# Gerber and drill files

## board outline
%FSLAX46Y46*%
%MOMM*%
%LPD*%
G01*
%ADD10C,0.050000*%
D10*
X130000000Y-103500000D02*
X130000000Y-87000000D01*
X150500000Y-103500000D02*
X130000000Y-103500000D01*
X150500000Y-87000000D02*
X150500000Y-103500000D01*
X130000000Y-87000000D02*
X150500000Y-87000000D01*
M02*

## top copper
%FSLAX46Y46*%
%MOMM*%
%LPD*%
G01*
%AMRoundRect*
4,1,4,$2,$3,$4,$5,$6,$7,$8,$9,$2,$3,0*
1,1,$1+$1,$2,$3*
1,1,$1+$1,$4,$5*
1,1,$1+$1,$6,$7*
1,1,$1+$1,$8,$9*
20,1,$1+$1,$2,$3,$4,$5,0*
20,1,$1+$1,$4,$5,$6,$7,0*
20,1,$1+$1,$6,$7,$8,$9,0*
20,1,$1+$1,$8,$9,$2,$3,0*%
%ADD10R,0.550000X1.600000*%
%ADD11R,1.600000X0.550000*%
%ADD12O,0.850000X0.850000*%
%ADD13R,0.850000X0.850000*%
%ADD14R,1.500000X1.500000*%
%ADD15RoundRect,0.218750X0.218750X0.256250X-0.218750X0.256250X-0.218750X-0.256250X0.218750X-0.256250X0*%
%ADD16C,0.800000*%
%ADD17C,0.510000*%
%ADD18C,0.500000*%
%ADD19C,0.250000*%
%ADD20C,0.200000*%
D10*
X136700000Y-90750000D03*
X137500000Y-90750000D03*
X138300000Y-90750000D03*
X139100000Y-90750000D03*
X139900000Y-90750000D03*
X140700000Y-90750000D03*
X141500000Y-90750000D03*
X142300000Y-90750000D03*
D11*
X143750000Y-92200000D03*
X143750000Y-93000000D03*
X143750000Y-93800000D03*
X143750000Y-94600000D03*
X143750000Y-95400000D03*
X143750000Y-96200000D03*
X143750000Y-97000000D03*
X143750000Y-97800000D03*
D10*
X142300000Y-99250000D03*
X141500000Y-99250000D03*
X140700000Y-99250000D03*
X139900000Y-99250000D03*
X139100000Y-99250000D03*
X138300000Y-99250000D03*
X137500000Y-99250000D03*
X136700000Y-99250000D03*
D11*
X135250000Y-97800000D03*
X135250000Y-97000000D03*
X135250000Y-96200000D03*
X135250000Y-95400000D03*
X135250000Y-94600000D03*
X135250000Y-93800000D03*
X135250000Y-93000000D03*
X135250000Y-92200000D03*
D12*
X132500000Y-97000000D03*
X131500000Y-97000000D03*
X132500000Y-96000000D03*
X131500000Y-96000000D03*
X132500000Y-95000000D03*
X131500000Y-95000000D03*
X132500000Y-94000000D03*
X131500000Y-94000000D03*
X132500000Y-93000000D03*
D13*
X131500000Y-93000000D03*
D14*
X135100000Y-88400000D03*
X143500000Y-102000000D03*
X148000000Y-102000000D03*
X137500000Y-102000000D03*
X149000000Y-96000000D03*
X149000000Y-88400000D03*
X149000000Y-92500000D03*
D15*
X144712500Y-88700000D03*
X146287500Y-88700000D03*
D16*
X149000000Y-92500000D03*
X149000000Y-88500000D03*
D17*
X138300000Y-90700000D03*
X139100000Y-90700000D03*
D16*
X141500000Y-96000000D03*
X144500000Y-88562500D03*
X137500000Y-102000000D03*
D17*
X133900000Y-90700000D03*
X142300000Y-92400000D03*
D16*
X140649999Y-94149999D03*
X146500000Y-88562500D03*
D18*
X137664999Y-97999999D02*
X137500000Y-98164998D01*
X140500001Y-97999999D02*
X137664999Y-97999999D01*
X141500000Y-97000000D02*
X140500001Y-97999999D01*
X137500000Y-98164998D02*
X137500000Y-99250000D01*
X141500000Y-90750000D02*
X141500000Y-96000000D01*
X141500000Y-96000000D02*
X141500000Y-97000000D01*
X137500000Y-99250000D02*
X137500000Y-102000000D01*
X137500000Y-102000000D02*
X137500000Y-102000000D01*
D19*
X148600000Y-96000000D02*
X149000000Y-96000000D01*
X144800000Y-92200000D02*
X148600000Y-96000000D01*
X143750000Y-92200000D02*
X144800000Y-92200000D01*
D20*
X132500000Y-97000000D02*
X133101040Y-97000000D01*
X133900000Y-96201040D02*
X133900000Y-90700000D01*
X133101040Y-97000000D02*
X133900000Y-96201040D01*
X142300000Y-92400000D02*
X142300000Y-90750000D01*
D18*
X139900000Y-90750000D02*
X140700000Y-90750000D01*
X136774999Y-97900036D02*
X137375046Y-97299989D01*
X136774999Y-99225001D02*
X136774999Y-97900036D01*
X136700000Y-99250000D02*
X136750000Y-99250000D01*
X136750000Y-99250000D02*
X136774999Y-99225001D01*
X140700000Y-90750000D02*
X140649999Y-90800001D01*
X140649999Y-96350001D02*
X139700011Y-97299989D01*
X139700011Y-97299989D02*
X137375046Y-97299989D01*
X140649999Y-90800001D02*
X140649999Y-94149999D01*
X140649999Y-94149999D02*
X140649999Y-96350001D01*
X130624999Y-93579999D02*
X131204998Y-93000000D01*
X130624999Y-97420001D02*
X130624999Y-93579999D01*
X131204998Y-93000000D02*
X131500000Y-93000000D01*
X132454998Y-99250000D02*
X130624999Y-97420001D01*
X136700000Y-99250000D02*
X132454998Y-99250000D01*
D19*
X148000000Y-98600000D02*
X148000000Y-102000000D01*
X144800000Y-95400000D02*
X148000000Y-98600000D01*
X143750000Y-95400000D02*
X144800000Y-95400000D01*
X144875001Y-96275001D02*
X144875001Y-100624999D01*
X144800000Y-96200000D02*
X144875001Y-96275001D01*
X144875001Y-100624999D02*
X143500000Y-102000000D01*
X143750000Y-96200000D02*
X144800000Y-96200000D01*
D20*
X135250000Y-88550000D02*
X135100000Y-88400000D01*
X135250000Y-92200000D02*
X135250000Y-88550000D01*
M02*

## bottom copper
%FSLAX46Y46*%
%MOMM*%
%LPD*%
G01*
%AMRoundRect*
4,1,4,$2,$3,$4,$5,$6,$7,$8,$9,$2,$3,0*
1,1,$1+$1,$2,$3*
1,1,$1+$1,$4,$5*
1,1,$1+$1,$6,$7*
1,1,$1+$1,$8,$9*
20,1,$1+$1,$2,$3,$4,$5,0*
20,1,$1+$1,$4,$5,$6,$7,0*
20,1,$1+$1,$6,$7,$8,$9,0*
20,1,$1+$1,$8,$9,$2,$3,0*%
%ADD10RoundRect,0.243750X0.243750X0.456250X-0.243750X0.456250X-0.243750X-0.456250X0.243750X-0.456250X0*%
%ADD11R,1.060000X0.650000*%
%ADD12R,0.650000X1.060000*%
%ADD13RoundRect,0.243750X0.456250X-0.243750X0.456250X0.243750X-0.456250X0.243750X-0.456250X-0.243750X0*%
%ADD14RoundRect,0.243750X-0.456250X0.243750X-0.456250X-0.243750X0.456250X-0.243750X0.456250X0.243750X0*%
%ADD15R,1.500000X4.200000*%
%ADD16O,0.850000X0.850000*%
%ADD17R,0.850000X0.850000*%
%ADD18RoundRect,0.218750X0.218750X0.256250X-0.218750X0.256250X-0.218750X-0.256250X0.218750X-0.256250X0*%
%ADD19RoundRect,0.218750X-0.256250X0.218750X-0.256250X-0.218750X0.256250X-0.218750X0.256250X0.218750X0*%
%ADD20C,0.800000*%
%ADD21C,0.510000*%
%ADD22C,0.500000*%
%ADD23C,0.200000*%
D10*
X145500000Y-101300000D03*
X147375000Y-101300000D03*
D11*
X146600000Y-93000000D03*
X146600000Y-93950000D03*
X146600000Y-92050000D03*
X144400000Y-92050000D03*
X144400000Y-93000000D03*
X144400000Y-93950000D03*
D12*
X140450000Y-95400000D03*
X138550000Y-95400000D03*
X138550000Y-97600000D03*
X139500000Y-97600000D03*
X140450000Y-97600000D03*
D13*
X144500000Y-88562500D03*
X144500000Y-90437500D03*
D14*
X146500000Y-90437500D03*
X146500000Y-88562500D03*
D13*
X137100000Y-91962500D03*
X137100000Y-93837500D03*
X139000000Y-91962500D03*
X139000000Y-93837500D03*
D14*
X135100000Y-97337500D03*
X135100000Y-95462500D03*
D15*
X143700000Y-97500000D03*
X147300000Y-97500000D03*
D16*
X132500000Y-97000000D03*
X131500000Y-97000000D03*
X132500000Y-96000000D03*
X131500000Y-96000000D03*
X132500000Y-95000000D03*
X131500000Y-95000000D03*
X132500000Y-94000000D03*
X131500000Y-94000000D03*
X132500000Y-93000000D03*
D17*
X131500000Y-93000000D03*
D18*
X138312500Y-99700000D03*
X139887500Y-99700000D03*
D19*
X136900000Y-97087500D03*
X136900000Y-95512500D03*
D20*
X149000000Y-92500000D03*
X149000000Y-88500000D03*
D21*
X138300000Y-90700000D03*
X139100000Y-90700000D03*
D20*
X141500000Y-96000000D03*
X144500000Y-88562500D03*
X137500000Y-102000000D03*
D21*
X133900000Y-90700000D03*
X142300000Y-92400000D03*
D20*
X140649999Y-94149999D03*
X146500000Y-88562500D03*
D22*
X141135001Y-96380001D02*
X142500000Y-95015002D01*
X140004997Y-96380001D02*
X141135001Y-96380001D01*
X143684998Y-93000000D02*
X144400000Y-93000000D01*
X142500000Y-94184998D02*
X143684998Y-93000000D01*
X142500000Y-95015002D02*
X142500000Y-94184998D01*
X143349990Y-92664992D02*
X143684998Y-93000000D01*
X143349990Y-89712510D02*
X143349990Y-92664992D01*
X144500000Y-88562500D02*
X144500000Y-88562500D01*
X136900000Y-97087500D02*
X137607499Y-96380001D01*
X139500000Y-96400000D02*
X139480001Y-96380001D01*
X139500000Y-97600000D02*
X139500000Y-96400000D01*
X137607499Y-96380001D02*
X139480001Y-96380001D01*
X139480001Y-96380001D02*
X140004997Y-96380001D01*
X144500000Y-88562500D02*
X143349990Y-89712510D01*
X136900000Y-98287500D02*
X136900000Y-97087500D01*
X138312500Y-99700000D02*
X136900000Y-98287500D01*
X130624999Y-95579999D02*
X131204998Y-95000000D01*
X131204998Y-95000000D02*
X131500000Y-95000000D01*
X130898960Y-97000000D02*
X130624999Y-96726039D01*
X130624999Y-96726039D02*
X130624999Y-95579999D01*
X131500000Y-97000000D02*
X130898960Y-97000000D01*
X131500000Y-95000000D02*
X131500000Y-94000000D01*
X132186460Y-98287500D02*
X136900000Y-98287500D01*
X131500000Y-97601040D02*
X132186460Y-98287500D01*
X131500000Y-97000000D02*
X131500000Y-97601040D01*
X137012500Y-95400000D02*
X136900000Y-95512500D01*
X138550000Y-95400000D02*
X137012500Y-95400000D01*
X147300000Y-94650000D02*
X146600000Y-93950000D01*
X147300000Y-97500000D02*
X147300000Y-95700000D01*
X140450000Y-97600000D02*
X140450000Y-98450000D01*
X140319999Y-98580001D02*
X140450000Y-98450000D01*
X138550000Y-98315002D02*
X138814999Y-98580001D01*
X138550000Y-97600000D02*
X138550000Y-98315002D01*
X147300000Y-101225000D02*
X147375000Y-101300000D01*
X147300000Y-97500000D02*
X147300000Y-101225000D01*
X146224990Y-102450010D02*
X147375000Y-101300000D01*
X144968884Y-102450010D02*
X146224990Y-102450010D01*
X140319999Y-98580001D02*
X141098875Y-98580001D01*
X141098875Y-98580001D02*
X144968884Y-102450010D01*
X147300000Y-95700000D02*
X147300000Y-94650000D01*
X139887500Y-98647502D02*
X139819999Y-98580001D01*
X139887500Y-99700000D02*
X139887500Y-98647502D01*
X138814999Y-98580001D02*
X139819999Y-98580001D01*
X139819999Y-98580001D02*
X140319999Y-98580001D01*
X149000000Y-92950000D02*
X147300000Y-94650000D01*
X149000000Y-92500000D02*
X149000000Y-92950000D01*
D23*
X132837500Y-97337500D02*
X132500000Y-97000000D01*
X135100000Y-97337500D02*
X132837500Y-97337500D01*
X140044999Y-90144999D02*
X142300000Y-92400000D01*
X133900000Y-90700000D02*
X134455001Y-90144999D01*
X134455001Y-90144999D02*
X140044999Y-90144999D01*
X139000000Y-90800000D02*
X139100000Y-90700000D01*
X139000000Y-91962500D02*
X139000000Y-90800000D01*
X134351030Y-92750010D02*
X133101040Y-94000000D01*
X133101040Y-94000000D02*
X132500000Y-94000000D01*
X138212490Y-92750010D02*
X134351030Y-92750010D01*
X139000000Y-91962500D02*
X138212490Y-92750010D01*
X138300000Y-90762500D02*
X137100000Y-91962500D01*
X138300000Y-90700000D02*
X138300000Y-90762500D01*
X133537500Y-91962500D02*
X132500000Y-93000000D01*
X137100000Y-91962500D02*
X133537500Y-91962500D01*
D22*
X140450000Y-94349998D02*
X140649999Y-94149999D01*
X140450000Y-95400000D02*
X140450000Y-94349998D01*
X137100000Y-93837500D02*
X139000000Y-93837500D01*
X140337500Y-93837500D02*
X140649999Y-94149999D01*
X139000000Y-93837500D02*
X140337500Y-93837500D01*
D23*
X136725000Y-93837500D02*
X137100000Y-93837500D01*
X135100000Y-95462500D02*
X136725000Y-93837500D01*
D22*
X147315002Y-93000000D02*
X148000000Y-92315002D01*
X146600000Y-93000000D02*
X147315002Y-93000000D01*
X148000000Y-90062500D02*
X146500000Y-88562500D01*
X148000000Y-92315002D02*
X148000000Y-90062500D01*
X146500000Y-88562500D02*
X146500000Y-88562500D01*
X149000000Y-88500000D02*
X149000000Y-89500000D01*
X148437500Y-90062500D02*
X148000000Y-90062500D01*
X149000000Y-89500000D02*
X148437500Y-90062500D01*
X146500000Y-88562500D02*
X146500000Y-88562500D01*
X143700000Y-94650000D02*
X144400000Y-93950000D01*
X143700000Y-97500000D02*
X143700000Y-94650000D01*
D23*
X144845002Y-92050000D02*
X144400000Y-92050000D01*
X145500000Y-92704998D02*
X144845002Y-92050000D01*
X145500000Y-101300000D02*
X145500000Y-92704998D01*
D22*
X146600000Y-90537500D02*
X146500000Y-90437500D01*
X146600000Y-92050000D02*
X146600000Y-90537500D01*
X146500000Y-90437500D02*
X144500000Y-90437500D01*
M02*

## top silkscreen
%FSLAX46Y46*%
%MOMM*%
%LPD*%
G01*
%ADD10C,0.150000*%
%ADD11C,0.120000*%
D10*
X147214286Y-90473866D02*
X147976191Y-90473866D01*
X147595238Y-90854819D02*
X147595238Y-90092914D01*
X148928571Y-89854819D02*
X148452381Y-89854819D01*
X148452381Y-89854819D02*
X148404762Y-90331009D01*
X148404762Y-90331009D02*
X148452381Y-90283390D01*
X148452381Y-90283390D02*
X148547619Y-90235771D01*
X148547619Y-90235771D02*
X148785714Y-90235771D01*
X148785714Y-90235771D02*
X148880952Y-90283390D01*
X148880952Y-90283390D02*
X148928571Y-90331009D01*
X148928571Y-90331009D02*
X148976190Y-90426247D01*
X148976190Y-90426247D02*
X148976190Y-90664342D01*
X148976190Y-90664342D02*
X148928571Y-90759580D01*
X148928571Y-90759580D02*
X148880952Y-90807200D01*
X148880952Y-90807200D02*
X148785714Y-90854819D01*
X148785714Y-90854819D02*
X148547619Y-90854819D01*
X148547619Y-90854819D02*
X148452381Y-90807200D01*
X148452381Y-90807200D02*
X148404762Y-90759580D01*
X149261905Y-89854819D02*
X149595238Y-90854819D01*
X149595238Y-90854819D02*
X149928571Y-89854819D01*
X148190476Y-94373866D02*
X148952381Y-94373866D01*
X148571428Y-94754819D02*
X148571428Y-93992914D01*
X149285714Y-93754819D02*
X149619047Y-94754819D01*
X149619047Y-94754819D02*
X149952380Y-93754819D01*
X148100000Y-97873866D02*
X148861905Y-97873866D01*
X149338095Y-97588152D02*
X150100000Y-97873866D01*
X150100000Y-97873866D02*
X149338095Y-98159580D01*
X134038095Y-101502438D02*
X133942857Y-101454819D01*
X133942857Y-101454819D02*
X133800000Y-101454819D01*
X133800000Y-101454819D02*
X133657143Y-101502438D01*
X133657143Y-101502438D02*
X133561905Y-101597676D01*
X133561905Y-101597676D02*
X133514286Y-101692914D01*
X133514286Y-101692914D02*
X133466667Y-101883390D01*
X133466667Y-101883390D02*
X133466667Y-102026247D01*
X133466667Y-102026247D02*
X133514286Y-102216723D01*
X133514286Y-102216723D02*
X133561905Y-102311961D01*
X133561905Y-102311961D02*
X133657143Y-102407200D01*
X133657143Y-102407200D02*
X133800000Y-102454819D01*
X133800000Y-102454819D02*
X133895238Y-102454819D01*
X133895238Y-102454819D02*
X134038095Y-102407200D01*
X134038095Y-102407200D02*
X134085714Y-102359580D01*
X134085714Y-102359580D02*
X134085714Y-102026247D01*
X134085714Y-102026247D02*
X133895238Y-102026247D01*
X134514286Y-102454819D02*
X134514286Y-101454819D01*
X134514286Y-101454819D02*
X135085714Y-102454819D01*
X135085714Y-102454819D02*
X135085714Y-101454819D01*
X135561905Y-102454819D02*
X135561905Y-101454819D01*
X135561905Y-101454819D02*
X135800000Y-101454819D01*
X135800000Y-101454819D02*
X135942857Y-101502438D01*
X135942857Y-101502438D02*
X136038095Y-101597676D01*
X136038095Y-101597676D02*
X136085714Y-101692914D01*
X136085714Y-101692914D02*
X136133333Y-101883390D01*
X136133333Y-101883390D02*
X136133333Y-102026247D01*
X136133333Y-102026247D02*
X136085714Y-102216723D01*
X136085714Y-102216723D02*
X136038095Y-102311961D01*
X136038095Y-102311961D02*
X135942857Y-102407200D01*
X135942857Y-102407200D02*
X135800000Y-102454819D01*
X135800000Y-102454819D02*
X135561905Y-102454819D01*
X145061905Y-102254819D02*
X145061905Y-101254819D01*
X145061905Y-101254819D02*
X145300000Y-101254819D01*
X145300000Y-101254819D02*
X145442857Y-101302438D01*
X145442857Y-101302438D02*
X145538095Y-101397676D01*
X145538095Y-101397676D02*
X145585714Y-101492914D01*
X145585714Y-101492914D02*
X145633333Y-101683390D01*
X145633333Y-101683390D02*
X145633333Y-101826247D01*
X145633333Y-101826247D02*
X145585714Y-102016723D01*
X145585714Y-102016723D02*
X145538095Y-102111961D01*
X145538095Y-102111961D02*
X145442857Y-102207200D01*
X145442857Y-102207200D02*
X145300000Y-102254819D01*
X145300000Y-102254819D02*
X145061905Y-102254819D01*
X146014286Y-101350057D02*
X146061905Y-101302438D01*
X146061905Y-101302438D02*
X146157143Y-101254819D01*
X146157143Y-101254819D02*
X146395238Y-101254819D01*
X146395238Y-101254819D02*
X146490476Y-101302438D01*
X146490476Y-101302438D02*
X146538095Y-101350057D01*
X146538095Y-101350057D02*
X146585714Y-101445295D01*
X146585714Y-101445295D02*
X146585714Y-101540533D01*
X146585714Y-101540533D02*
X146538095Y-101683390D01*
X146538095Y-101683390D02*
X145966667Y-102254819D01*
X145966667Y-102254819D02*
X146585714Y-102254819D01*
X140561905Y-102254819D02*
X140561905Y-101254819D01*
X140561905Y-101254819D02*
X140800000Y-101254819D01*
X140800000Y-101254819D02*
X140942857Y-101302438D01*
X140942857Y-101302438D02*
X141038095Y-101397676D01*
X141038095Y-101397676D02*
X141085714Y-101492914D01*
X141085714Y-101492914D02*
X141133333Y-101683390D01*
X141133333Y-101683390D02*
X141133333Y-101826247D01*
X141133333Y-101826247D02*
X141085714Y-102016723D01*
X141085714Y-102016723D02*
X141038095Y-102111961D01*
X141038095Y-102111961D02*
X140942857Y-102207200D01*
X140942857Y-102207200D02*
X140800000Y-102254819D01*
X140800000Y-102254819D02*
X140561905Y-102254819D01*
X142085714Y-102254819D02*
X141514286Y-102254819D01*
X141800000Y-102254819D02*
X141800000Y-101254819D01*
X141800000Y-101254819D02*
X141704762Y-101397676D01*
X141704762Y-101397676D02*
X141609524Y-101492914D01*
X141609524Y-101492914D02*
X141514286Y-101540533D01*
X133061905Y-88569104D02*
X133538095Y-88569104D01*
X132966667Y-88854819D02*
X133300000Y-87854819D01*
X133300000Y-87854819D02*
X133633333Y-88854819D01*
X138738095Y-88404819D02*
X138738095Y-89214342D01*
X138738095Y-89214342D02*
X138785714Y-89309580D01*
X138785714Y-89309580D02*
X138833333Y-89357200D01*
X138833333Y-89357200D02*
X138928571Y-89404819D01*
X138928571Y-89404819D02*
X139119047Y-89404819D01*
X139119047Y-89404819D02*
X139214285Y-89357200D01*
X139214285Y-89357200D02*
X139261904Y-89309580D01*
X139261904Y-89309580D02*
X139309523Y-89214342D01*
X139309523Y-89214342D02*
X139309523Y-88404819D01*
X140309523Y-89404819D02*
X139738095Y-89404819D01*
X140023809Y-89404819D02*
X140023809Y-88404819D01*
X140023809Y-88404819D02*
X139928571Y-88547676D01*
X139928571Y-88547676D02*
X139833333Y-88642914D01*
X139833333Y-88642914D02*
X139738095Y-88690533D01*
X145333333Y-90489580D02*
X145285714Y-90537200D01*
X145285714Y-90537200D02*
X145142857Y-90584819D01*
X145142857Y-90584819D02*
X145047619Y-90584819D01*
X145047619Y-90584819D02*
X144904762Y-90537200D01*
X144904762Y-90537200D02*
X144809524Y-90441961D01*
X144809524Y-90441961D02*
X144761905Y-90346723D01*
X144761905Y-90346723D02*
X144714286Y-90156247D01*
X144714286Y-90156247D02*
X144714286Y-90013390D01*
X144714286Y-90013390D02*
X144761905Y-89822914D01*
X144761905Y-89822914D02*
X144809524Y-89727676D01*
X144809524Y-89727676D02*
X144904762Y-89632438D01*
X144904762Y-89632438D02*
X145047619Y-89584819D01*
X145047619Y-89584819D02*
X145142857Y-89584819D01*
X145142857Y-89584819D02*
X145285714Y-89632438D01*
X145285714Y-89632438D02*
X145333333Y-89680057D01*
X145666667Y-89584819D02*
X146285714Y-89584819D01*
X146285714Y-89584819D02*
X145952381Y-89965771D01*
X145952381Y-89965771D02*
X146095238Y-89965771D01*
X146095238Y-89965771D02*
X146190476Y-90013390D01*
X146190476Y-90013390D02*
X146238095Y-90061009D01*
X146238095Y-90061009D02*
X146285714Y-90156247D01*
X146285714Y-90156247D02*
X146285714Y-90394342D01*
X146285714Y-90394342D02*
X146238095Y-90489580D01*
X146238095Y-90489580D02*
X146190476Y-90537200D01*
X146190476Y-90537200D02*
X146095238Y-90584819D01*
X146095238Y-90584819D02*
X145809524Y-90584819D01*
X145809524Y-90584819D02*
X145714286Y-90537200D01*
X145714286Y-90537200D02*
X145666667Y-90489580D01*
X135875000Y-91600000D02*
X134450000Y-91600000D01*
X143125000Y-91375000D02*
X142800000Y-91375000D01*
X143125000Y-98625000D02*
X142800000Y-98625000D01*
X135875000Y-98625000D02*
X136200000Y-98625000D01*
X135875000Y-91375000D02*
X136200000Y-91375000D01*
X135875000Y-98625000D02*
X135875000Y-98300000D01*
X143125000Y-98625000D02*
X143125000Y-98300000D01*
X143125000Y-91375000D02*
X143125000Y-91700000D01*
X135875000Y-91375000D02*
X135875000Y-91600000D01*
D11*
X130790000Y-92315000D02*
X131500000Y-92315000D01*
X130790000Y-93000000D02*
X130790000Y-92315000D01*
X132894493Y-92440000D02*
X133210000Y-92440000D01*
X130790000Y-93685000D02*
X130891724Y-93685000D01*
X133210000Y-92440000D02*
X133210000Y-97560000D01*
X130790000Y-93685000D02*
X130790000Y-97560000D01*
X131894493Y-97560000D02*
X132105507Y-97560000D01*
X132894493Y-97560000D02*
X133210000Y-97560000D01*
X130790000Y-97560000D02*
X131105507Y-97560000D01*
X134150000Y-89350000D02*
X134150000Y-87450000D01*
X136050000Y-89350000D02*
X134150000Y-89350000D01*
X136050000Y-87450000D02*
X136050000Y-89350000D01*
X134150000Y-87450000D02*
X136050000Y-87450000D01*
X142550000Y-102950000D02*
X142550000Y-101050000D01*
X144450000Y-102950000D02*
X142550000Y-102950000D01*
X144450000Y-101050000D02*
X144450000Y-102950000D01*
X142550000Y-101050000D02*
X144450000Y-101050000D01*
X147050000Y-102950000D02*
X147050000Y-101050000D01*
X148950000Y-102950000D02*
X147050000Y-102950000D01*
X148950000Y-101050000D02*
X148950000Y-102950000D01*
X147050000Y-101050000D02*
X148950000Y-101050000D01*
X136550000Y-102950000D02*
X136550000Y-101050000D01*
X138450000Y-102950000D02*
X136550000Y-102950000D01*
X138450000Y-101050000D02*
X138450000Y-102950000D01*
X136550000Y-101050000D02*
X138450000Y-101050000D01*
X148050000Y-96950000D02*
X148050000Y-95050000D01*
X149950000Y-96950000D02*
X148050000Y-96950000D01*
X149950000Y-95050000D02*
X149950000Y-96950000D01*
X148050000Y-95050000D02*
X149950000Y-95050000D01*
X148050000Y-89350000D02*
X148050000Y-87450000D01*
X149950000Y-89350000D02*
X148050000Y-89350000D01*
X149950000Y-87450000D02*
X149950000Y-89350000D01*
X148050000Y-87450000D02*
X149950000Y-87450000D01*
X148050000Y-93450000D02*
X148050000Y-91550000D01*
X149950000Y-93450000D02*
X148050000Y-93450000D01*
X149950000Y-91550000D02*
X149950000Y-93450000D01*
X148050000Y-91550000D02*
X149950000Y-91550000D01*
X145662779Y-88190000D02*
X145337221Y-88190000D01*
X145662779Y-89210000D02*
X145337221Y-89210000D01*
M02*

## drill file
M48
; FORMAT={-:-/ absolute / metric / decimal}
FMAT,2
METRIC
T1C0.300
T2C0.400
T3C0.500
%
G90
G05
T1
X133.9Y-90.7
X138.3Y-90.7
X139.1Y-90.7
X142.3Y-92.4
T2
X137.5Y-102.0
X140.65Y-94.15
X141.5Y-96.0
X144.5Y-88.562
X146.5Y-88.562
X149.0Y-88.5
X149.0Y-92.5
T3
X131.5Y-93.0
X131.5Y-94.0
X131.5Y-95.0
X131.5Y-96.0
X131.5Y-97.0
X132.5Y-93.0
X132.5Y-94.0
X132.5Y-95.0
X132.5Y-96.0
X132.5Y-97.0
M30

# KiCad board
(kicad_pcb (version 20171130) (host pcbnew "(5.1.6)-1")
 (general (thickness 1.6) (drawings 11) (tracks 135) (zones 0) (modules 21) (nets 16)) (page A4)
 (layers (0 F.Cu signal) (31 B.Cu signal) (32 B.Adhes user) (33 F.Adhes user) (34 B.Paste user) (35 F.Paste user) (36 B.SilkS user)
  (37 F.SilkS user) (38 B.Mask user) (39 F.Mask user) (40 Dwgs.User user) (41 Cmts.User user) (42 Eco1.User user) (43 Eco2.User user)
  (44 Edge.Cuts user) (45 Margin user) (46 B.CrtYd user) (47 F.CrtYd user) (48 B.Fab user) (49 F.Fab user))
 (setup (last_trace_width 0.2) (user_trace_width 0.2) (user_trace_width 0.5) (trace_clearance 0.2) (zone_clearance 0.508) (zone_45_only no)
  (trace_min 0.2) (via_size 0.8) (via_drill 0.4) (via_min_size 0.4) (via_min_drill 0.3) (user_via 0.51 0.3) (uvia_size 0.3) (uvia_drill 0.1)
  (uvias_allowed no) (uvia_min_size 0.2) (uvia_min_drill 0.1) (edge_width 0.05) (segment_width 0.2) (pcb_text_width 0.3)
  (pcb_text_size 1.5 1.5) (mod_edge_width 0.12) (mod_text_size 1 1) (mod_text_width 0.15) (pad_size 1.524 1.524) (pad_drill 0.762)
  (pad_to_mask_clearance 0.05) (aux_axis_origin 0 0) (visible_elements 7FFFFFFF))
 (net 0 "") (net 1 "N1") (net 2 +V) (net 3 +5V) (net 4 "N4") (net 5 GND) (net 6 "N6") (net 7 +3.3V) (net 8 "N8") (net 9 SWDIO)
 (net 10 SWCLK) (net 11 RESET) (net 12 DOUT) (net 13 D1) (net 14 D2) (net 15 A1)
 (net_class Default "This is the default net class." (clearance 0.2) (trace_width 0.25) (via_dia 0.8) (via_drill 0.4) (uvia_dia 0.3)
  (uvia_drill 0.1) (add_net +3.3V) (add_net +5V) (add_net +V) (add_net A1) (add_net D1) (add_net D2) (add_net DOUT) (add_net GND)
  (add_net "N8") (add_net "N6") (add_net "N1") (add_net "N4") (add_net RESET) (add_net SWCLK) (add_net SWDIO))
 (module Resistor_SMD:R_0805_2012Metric (layer B.Cu) (at 146.4375 101.3 180)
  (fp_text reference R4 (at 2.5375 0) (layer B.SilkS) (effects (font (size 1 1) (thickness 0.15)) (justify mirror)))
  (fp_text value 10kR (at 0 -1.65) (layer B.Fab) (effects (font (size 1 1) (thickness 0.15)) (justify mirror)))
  (pad 2 smd roundrect (at 0.9375 0 180) (size 0.975 1.4) (layers B.Cu B.Paste B.Mask) (roundrect_rratio 0.25) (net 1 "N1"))
  (pad 1 smd roundrect (at -0.9375 0 180) (size 0.975 1.4) (layers B.Cu B.Paste B.Mask) (roundrect_rratio 0.25) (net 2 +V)))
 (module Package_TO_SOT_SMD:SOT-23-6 (layer B.Cu) (at 145.5 93)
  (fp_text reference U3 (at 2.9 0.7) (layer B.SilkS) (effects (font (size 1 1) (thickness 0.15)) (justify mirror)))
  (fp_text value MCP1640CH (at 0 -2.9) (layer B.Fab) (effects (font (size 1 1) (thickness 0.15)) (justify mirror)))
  (pad 5 smd rect (at 1.1 0) (size 1.06 0.65) (layers B.Cu B.Paste B.Mask) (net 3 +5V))
  (pad 6 smd rect (at 1.1 0.95) (size 1.06 0.65) (layers B.Cu B.Paste B.Mask) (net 2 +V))
  (pad 4 smd rect (at 1.1 -0.95) (size 1.06 0.65) (layers B.Cu B.Paste B.Mask) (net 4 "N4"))
  (pad 3 smd rect (at -1.1 -0.95) (size 1.06 0.65) (layers B.Cu B.Paste B.Mask) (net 1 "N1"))
  (pad 2 smd rect (at -1.1 0) (size 1.06 0.65) (layers B.Cu B.Paste B.Mask) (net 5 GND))
  (pad 1 smd rect (at -1.1 0.95) (size 1.06 0.65) (layers B.Cu B.Paste B.Mask) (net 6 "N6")))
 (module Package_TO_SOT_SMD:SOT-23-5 (layer B.Cu) (at 139.5 96.5 90)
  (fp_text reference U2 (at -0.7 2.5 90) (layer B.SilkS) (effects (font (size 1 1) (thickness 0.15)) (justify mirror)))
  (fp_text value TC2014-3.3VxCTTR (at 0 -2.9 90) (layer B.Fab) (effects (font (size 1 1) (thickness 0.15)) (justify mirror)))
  (pad 5 smd rect (at 1.1 0.95 90) (size 1.06 0.65) (layers B.Cu B.Paste B.Mask) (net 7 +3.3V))
  (pad 4 smd rect (at 1.1 -0.95 90) (size 1.06 0.65) (layers B.Cu B.Paste B.Mask) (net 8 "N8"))
  (pad 3 smd rect (at -1.1 -0.95 90) (size 1.06 0.65) (layers B.Cu B.Paste B.Mask) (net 2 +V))
  (pad 2 smd rect (at -1.1 0 90) (size 1.06 0.65) (layers B.Cu B.Paste B.Mask) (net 5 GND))
  (pad 1 smd rect (at -1.1 0.95 90) (size 1.06 0.65) (layers B.Cu B.Paste B.Mask) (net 2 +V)))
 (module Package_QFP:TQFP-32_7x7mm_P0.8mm (layer F.Cu) (at 139.5 95)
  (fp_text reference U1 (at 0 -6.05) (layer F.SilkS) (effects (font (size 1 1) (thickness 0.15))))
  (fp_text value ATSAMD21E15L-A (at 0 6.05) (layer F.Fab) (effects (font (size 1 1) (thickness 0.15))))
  (fp_line (start -3.625 -3.4) (end -5.05 -3.4) (layer F.SilkS) (width 0.15))
  (fp_line (start 3.625 -3.625) (end 3.3 -3.625) (layer F.SilkS) (width 0.15))
  (fp_line (start 3.625 3.625) (end 3.3 3.625) (layer F.SilkS) (width 0.15))
  (fp_line (start -3.625 3.625) (end -3.3 3.625) (layer F.SilkS) (width 0.15))
  (fp_line (start -3.625 -3.625) (end -3.3 -3.625) (layer F.SilkS) (width 0.15))
  (fp_line (start -3.625 3.625) (end -3.625 3.3) (layer F.SilkS) (width 0.15))
  (fp_line (start 3.625 3.625) (end 3.625 3.3) (layer F.SilkS) (width 0.15))
  (fp_line (start 3.625 -3.625) (end 3.625 -3.3) (layer F.SilkS) (width 0.15))
  (fp_line (start -3.625 -3.625) (end -3.625 -3.4) (layer F.SilkS) (width 0.15))
  (pad 32 smd rect (at -2.8 -4.25 90) (size 1.6 0.55) (layers F.Cu F.Paste F.Mask))
  (pad 31 smd rect (at -2 -4.25 90) (size 1.6 0.55) (layers F.Cu F.Paste F.Mask))
  (pad 30 smd rect (at -1.2 -4.25 90) (size 1.6 0.55) (layers F.Cu F.Paste F.Mask) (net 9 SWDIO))
  (pad 29 smd rect (at -0.4 -4.25 90) (size 1.6 0.55) (layers F.Cu F.Paste F.Mask) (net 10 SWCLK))
  (pad 28 smd rect (at 0.4 -4.25 90) (size 1.6 0.55) (layers F.Cu F.Paste F.Mask) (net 7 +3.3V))
  (pad 27 smd rect (at 1.2 -4.25 90) (size 1.6 0.55) (layers F.Cu F.Paste F.Mask) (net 7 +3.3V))
  (pad 26 smd rect (at 2 -4.25 90) (size 1.6 0.55) (layers F.Cu F.Paste F.Mask) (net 5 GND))
  (pad 25 smd rect (at 2.8 -4.25 90) (size 1.6 0.55) (layers F.Cu F.Paste F.Mask) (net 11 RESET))
  (pad 24 smd rect (at 4.25 -2.8) (size 1.6 0.55) (layers F.Cu F.Paste F.Mask) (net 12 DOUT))
  (pad 23 smd rect (at 4.25 -2) (size 1.6 0.55) (layers F.Cu F.Paste F.Mask))
  (pad 22 smd rect (at 4.25 -1.2) (size 1.6 0.55) (layers F.Cu F.Paste F.Mask))
  (pad 21 smd rect (at 4.25 -0.4) (size 1.6 0.55) (layers F.Cu F.Paste F.Mask))
  (pad 20 smd rect (at 4.25 0.4) (size 1.6 0.55) (layers F.Cu F.Paste F.Mask) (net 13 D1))
  (pad 19 smd rect (at 4.25 1.2) (size 1.6 0.55) (layers F.Cu F.Paste F.Mask) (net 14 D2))
  (pad 18 smd rect (at 4.25 2) (size 1.6 0.55) (layers F.Cu F.Paste F.Mask))
  (pad 17 smd rect (at 4.25 2.8) (size 1.6 0.55) (layers F.Cu F.Paste F.Mask))
  (pad 16 smd rect (at 2.8 4.25 90) (size 1.6 0.55) (layers F.Cu F.Paste F.Mask))
  (pad 15 smd rect (at 2 4.25 90) (size 1.6 0.55) (layers F.Cu F.Paste F.Mask))
  (pad 14 smd rect (at 1.2 4.25 90) (size 1.6 0.55) (layers F.Cu F.Paste F.Mask))
  (pad 13 smd rect (at 0.4 4.25 90) (size 1.6 0.55) (layers F.Cu F.Paste F.Mask))
  (pad 12 smd rect (at -0.4 4.25 90) (size 1.6 0.55) (layers F.Cu F.Paste F.Mask))
  (pad 11 smd rect (at -1.2 4.25 90) (size 1.6 0.55) (layers F.Cu F.Paste F.Mask))
  (pad 10 smd rect (at -2 4.25 90) (size 1.6 0.55) (layers F.Cu F.Paste F.Mask) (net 5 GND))
  (pad 9 smd rect (at -2.8 4.25 90) (size 1.6 0.55) (layers F.Cu F.Paste F.Mask) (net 7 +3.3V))
  (pad 8 smd rect (at -4.25 2.8) (size 1.6 0.55) (layers F.Cu F.Paste F.Mask))
  (pad 7 smd rect (at -4.25 2) (size 1.6 0.55) (layers F.Cu F.Paste F.Mask))
  (pad 6 smd rect (at -4.25 1.2) (size 1.6 0.55) (layers F.Cu F.Paste F.Mask))
  (pad 5 smd rect (at -4.25 0.4) (size 1.6 0.55) (layers F.Cu F.Paste F.Mask))
  (pad 4 smd rect (at -4.25 -0.4) (size 1.6 0.55) (layers F.Cu F.Paste F.Mask))
  (pad 3 smd rect (at -4.25 -1.2) (size 1.6 0.55) (layers F.Cu F.Paste F.Mask))
  (pad 2 smd rect (at -4.25 -2) (size 1.6 0.55) (layers F.Cu F.Paste F.Mask))
  (pad 1 smd rect (at -4.25 -2.8) (size 1.6 0.55) (layers F.Cu F.Paste F.Mask) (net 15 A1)))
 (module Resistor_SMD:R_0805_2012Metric (layer B.Cu) (at 144.5 89.5 90)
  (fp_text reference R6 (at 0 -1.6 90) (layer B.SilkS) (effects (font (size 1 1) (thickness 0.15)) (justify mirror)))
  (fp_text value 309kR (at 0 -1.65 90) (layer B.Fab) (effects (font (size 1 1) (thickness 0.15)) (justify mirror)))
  (pad 2 smd roundrect (at 0.9375 0 90) (size 0.975 1.4) (layers B.Cu B.Paste B.Mask) (roundrect_rratio 0.25) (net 5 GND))
  (pad 1 smd roundrect (at -0.9375 0 90) (size 0.975 1.4) (layers B.Cu B.Paste B.Mask) (roundrect_rratio 0.25) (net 4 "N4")))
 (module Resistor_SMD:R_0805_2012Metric (layer B.Cu) (at 146.5 89.5 270)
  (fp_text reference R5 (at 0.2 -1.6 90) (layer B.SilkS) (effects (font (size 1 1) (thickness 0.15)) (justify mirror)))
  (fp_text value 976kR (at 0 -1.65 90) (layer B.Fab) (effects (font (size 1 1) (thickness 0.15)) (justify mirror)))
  (pad 2 smd roundrect (at 0.9375 0 270) (size 0.975 1.4) (layers B.Cu B.Paste B.Mask) (roundrect_rratio 0.25) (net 4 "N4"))
  (pad 1 smd roundrect (at -0.9375 0 270) (size 0.975 1.4) (layers B.Cu B.Paste B.Mask) (roundrect_rratio 0.25) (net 3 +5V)))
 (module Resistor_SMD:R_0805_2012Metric (layer B.Cu) (at 137.1 92.9 90)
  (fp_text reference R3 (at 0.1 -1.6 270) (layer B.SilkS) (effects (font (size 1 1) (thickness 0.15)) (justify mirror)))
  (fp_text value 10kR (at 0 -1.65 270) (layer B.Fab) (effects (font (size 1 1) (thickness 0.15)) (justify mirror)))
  (pad 2 smd roundrect (at 0.9375 0 90) (size 0.975 1.4) (layers B.Cu B.Paste B.Mask) (roundrect_rratio 0.25) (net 9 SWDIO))
  (pad 1 smd roundrect (at -0.9375 0 90) (size 0.975 1.4) (layers B.Cu B.Paste B.Mask) (roundrect_rratio 0.25) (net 7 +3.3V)))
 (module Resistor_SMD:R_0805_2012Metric (layer B.Cu) (at 139 92.9 90)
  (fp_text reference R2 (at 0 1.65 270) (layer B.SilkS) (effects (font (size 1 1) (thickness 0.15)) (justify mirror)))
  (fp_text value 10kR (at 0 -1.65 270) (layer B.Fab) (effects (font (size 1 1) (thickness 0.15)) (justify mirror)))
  (pad 2 smd roundrect (at 0.9375 0 90) (size 0.975 1.4) (layers B.Cu B.Paste B.Mask) (roundrect_rratio 0.25) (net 10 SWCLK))
  (pad 1 smd roundrect (at -0.9375 0 90) (size 0.975 1.4) (layers B.Cu B.Paste B.Mask) (roundrect_rratio 0.25) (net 7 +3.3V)))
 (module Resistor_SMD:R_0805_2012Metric (layer B.Cu) (at 135.1 96.4 270)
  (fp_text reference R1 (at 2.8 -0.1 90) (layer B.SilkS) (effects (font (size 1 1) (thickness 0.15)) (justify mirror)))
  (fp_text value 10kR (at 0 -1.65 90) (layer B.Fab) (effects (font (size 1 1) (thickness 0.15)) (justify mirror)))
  (pad 2 smd roundrect (at 0.9375 0 270) (size 0.975 1.4) (layers B.Cu B.Paste B.Mask) (roundrect_rratio 0.25) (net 11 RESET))
  (pad 1 smd roundrect (at -0.9375 0 270) (size 0.975 1.4) (layers B.Cu B.Paste B.Mask) (roundrect_rratio 0.25) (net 7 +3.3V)))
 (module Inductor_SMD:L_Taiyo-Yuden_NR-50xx (layer B.Cu) (at 145.5 97.5 180)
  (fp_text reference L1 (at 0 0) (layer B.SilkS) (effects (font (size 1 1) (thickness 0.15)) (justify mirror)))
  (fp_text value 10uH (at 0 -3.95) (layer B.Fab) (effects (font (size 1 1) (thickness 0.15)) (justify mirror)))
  (pad 2 smd rect (at 1.8 0 180) (size 1.5 4.2) (layers B.Cu B.Paste B.Mask) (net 6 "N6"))
  (pad 1 smd rect (at -1.8 0 180) (size 1.5 4.2) (layers B.Cu B.Paste B.Mask) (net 2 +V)))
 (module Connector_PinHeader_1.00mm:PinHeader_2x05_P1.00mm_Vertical (layer F.Cu) (at 131.5 93)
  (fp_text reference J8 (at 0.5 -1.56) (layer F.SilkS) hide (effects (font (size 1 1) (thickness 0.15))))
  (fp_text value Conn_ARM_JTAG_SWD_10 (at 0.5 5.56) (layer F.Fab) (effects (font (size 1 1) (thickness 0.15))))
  (fp_line (start -0.71 -0.685) (end 0 -0.685) (layer F.SilkS) (width 0.12))
  (fp_line (start -0.71 0) (end -0.71 -0.685) (layer F.SilkS) (width 0.12))
  (fp_line (start 1.394493 -0.56) (end 1.71 -0.56) (layer F.SilkS) (width 0.12))
  (fp_line (start -0.71 0.685) (end -0.608276 0.685) (layer F.SilkS) (width 0.12))
  (fp_line (start 1.71 -0.56) (end 1.71 4.56) (layer F.SilkS) (width 0.12))
  (fp_line (start -0.71 0.685) (end -0.71 4.56) (layer F.SilkS) (width 0.12))
  (fp_line (start 0.394493 4.56) (end 0.605507 4.56) (layer F.SilkS) (width 0.12))
  (fp_line (start 1.394493 4.56) (end 1.71 4.56) (layer F.SilkS) (width 0.12))
  (fp_line (start -0.71 4.56) (end -0.394493 4.56) (layer F.SilkS) (width 0.12))
  (pad 10 thru_hole oval (at 1 4) (size 0.85 0.85) (drill 0.5) (layers *.Cu *.Mask) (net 11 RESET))
  (pad 9 thru_hole oval (at 0 4) (size 0.85 0.85) (drill 0.5) (layers *.Cu *.Mask) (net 5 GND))
  (pad 8 thru_hole oval (at 1 3) (size 0.85 0.85) (drill 0.5) (layers *.Cu *.Mask))
  (pad 7 thru_hole oval (at 0 3) (size 0.85 0.85) (drill 0.5) (layers *.Cu *.Mask))
  (pad 6 thru_hole oval (at 1 2) (size 0.85 0.85) (drill 0.5) (layers *.Cu *.Mask))
  (pad 5 thru_hole oval (at 0 2) (size 0.85 0.85) (drill 0.5) (layers *.Cu *.Mask) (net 5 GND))
  (pad 4 thru_hole oval (at 1 1) (size 0.85 0.85) (drill 0.5) (layers *.Cu *.Mask) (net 10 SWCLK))
  (pad 3 thru_hole oval (at 0 1) (size 0.85 0.85) (drill 0.5) (layers *.Cu *.Mask) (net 5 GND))
  (pad 2 thru_hole oval (at 1 0) (size 0.85 0.85) (drill 0.5) (layers *.Cu *.Mask) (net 9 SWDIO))
  (pad 1 thru_hole rect (at 0 0) (size 0.85 0.85) (drill 0.5) (layers *.Cu *.Mask) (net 7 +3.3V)))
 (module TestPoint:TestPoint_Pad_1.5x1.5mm (layer F.Cu) (at 135.1 88.4)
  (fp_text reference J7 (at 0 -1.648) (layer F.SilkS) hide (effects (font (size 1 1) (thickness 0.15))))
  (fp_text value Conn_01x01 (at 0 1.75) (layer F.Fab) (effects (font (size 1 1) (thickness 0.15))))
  (fp_line (start -0.95 0.95) (end -0.95 -0.95) (layer F.SilkS) (width 0.12))
  (fp_line (start 0.95 0.95) (end -0.95 0.95) (layer F.SilkS) (width 0.12))
  (fp_line (start 0.95 -0.95) (end 0.95 0.95) (layer F.SilkS) (width 0.12))
  (fp_line (start -0.95 -0.95) (end 0.95 -0.95) (layer F.SilkS) (width 0.12))
  (pad 1 smd rect (at 0 0) (size 1.5 1.5) (layers F.Cu F.Mask) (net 15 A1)))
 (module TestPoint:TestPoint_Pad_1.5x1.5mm (layer F.Cu) (at 143.5 102)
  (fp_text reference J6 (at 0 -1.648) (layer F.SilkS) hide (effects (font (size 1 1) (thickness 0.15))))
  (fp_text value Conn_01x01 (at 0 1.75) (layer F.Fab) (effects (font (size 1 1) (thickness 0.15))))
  (fp_line (start -0.95 0.95) (end -0.95 -0.95) (layer F.SilkS) (width 0.12))
  (fp_line (start 0.95 0.95) (end -0.95 0.95) (layer F.SilkS) (width 0.12))
  (fp_line (start 0.95 -0.95) (end 0.95 0.95) (layer F.SilkS) (width 0.12))
  (fp_line (start -0.95 -0.95) (end 0.95 -0.95) (layer F.SilkS) (width 0.12))
  (pad 1 smd rect (at 0 0) (size 1.5 1.5) (layers F.Cu F.Mask) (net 14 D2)))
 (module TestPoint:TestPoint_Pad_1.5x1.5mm (layer F.Cu) (at 148 102)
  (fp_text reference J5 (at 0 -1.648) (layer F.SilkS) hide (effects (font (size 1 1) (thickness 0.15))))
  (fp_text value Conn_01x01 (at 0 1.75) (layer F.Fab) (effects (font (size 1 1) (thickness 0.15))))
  (fp_line (start -0.95 0.95) (end -0.95 -0.95) (layer F.SilkS) (width 0.12))
  (fp_line (start 0.95 0.95) (end -0.95 0.95) (layer F.SilkS) (width 0.12))
  (fp_line (start 0.95 -0.95) (end 0.95 0.95) (layer F.SilkS) (width 0.12))
  (fp_line (start -0.95 -0.95) (end 0.95 -0.95) (layer F.SilkS) (width 0.12))
  (pad 1 smd rect (at 0 0) (size 1.5 1.5) (layers F.Cu F.Mask) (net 13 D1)))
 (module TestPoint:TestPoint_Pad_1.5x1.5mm (layer F.Cu) (at 137.5 102)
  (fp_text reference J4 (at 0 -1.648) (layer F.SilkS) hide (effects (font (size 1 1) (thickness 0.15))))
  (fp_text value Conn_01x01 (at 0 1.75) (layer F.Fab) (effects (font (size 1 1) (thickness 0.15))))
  (fp_line (start -0.95 0.95) (end -0.95 -0.95) (layer F.SilkS) (width 0.12))
  (fp_line (start 0.95 0.95) (end -0.95 0.95) (layer F.SilkS) (width 0.12))
  (fp_line (start 0.95 -0.95) (end 0.95 0.95) (layer F.SilkS) (width 0.12))
  (fp_line (start -0.95 -0.95) (end 0.95 -0.95) (layer F.SilkS) (width 0.12))
  (pad 1 smd rect (at 0 0) (size 1.5 1.5) (layers F.Cu F.Mask) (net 5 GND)))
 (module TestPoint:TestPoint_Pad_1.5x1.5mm (layer F.Cu) (at 149 96)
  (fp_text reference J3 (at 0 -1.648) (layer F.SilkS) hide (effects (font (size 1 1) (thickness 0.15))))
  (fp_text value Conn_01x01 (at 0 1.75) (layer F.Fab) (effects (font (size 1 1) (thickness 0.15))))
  (fp_line (start -0.95 0.95) (end -0.95 -0.95) (layer F.SilkS) (width 0.12))
  (fp_line (start 0.95 0.95) (end -0.95 0.95) (layer F.SilkS) (width 0.12))
  (fp_line (start 0.95 -0.95) (end 0.95 0.95) (layer F.SilkS) (width 0.12))
  (fp_line (start -0.95 -0.95) (end 0.95 -0.95) (layer F.SilkS) (width 0.12))
  (pad 1 smd rect (at 0 0) (size 1.5 1.5) (layers F.Cu F.Mask) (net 12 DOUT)))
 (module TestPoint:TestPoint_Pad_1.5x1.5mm (layer F.Cu) (at 149 88.4)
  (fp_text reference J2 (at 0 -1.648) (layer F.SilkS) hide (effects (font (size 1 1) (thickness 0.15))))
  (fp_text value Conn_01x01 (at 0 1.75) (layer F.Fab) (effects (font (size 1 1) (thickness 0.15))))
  (fp_line (start -0.95 0.95) (end -0.95 -0.95) (layer F.SilkS) (width 0.12))
  (fp_line (start 0.95 0.95) (end -0.95 0.95) (layer F.SilkS) (width 0.12))
  (fp_line (start 0.95 -0.95) (end 0.95 0.95) (layer F.SilkS) (width 0.12))
  (fp_line (start -0.95 -0.95) (end 0.95 -0.95) (layer F.SilkS) (width 0.12))
  (pad 1 smd rect (at 0 0) (size 1.5 1.5) (layers F.Cu F.Mask) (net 3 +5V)))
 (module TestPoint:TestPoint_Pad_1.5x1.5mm (layer F.Cu) (at 149 92.5)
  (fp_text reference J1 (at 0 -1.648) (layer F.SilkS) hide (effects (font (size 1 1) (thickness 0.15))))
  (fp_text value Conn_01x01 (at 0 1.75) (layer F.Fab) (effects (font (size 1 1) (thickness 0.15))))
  (fp_line (start -0.95 0.95) (end -0.95 -0.95) (layer F.SilkS) (width 0.12))
  (fp_line (start 0.95 0.95) (end -0.95 0.95) (layer F.SilkS) (width 0.12))
  (fp_line (start 0.95 -0.95) (end 0.95 0.95) (layer F.SilkS) (width 0.12))
  (fp_line (start -0.95 -0.95) (end 0.95 -0.95) (layer F.SilkS) (width 0.12))
  (pad 1 smd rect (at 0 0) (size 1.5 1.5) (layers F.Cu F.Mask) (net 2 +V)))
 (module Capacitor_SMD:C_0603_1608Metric (layer F.Cu) (at 145.5 88.7 180)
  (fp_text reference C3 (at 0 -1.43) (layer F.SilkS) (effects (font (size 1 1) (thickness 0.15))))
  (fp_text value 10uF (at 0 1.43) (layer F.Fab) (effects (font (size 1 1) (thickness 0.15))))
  (fp_line (start -0.162779 0.51) (end 0.162779 0.51) (layer F.SilkS) (width 0.12))
  (fp_line (start -0.162779 -0.51) (end 0.162779 -0.51) (layer F.SilkS) (width 0.12))
  (pad 2 smd roundrect (at 0.7875 0 180) (size 0.875 0.95) (layers F.Cu F.Paste F.Mask) (roundrect_rratio 0.25) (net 5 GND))
  (pad 1 smd roundrect (at -0.7875 0 180) (size 0.875 0.95) (layers F.Cu F.Paste F.Mask) (roundrect_rratio 0.25) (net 3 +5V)))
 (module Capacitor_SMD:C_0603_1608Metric (layer B.Cu) (at 139.1 99.7 180)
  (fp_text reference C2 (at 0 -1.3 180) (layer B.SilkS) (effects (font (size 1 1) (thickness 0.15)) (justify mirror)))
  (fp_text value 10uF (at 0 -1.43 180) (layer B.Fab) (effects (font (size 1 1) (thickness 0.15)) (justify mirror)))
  (pad 2 smd roundrect (at 0.7875 0 180) (size 0.875 0.95) (layers B.Cu B.Paste B.Mask) (roundrect_rratio 0.25) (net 5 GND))
  (pad 1 smd roundrect (at -0.7875 0 180) (size 0.875 0.95) (layers B.Cu B.Paste B.Mask) (roundrect_rratio 0.25) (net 2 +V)))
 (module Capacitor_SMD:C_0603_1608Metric (layer B.Cu) (at 136.9 96.3 270)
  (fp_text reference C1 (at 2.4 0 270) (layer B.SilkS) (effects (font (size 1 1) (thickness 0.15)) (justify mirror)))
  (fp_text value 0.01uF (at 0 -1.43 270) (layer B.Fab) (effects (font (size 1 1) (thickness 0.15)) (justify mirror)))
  (pad 2 smd roundrect (at 0.7875 0 270) (size 0.875 0.95) (layers B.Cu B.Paste B.Mask) (roundrect_rratio 0.25) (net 5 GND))
  (pad 1 smd roundrect (at -0.7875 0 270) (size 0.875 0.95) (layers B.Cu B.Paste B.Mask) (roundrect_rratio 0.25) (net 8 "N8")))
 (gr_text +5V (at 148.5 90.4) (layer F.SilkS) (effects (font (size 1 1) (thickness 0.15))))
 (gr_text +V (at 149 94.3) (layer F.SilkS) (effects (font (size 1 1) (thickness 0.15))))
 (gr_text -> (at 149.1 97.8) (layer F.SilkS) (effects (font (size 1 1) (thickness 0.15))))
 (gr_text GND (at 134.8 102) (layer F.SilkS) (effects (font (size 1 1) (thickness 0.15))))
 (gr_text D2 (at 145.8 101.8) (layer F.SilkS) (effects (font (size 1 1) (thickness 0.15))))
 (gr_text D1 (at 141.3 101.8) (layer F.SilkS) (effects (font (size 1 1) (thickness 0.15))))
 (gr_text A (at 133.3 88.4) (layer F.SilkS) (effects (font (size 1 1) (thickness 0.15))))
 (gr_line (start 130 103.5) (end 130 87) (layer Edge.Cuts) (width 0.05))
 (gr_line (start 150.5 103.5) (end 130 103.5) (layer Edge.Cuts) (width 0.05))
 (gr_line (start 150.5 87) (end 150.5 103.5) (layer Edge.Cuts) (width 0.05))
 (gr_line (start 130 87) (end 150.5 87) (layer Edge.Cuts) (width 0.05))
 (via (at 149 92.5) (size 0.8) (drill 0.4) (layers F.Cu B.Cu) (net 2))
 (via (at 149 88.5) (size 0.8) (drill 0.4) (layers F.Cu B.Cu) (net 3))
 (via (at 138.3 90.7) (size 0.51) (drill 0.3) (layers F.Cu B.Cu) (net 9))
 (via (at 139.1 90.7) (size 0.51) (drill 0.3) (layers F.Cu B.Cu) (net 10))
 (segment (start 141.135001 96.380001) (end 142.5 95.015002) (width 0.5) (layer B.Cu) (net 5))
 (segment (start 140.004997 96.380001) (end 141.135001 96.380001) (width 0.5) (layer B.Cu) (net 5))
 (segment (start 143.684998 93) (end 144.4 93) (width 0.5) (layer B.Cu) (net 5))
 (segment (start 142.5 94.184998) (end 143.684998 93) (width 0.5) (layer B.Cu) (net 5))
 (segment (start 142.5 95.015002) (end 142.5 94.184998) (width 0.5) (layer B.Cu) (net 5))
 (segment (start 137.664999 97.999999) (end 137.5 98.164998) (width 0.5) (layer F.Cu) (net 5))
 (segment (start 140.500001 97.999999) (end 137.664999 97.999999) (width 0.5) (layer F.Cu) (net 5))
 (segment (start 141.5 97) (end 140.500001 97.999999) (width 0.5) (layer F.Cu) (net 5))
 (segment (start 137.5 98.164998) (end 137.5 99.25) (width 0.5) (layer F.Cu) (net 5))
 (segment (start 141.5 90.75) (end 141.5 96) (width 0.5) (layer F.Cu) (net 5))
 (segment (start 141.5 96) (end 141.5 97) (width 0.5) (layer F.Cu) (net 5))
 (via (at 141.5 96) (size 0.8) (drill 0.4) (layers F.Cu B.Cu) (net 5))
 (segment (start 143.34999 92.664992) (end 143.684998 93) (width 0.5) (layer B.Cu) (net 5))
 (segment (start 143.34999 89.71251) (end 143.34999 92.664992) (width 0.5) (layer B.Cu) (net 5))
 (segment (start 144.5 88.5625) (end 144.5 88.5625) (width 0.5) (layer B.Cu) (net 5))
 (segment (start 136.9 97.0875) (end 137.607499 96.380001) (width 0.5) (layer B.Cu) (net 5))
 (segment (start 139.5 96.4) (end 139.480001 96.380001) (width 0.5) (layer B.Cu) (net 5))
 (segment (start 139.5 97.6) (end 139.5 96.4) (width 0.5) (layer B.Cu) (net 5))
 (segment (start 137.607499 96.380001) (end 139.480001 96.380001) (width 0.5) (layer B.Cu) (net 5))
 (segment (start 139.480001 96.380001) (end 140.004997 96.380001) (width 0.5) (layer B.Cu) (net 5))
 (segment (start 144.5 88.5625) (end 143.34999 89.71251) (width 0.5) (layer B.Cu) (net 5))
 (via (at 144.5 88.5625) (size 0.8) (drill 0.4) (layers F.Cu B.Cu) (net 5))
 (segment (start 136.9 98.2875) (end 136.9 97.0875) (width 0.5) (layer B.Cu) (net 5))
 (segment (start 138.3125 99.7) (end 136.9 98.2875) (width 0.5) (layer B.Cu) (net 5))
 (segment (start 130.624999 95.579999) (end 131.204998 95) (width 0.5) (layer B.Cu) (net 5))
 (segment (start 131.204998 95) (end 131.5 95) (width 0.5) (layer B.Cu) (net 5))
 (segment (start 130.89896 97) (end 130.624999 96.726039) (width 0.5) (layer B.Cu) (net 5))
 (segment (start 130.624999 96.726039) (end 130.624999 95.579999) (width 0.5) (layer B.Cu) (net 5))
 (segment (start 131.5 97) (end 130.89896 97) (width 0.5) (layer B.Cu) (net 5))
 (segment (start 131.5 95) (end 131.5 94) (width 0.5) (layer B.Cu) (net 5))
 (segment (start 132.18646 98.2875) (end 136.9 98.2875) (width 0.5) (layer B.Cu) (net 5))
 (segment (start 131.5 97.60104) (end 132.18646 98.2875) (width 0.5) (layer B.Cu) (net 5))
 (segment (start 131.5 97) (end 131.5 97.60104) (width 0.5) (layer B.Cu) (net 5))
 (segment (start 137.5 99.25) (end 137.5 102) (width 0.5) (layer F.Cu) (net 5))
 (segment (start 137.5 102) (end 137.5 102) (width 0.5) (layer F.Cu) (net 5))
 (via (at 137.5 102) (size 0.8) (drill 0.4) (layers F.Cu B.Cu) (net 5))
 (segment (start 137.0125 95.4) (end 136.9 95.5125) (width 0.5) (layer B.Cu) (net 8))
 (segment (start 138.55 95.4) (end 137.0125 95.4) (width 0.5) (layer B.Cu) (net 8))
 (segment (start 147.3 94.65) (end 146.6 93.95) (width 0.5) (layer B.Cu) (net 2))
 (segment (start 147.3 97.5) (end 147.3 95.7) (width 0.5) (layer B.Cu) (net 2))
 (segment (start 140.45 97.6) (end 140.45 98.45) (width 0.5) (layer B.Cu) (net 2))
 (segment (start 140.319999 98.580001) (end 140.45 98.45) (width 0.5) (layer B.Cu) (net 2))
 (segment (start 138.55 98.315002) (end 138.814999 98.580001) (width 0.5) (layer B.Cu) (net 2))
 (segment (start 138.55 97.6) (end 138.55 98.315002) (width 0.5) (layer B.Cu) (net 2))
 (segment (start 147.3 101.225) (end 147.375 101.3) (width 0.5) (layer B.Cu) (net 2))
 (segment (start 147.3 97.5) (end 147.3 101.225) (width 0.5) (layer B.Cu) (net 2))
 (segment (start 146.22499 102.45001) (end 147.375 101.3) (width 0.5) (layer B.Cu) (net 2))
 (segment (start 144.968884 102.45001) (end 146.22499 102.45001) (width 0.5) (layer B.Cu) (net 2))
 (segment (start 140.319999 98.580001) (end 141.098875 98.580001) (width 0.5) (layer B.Cu) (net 2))
 (segment (start 141.098875 98.580001) (end 144.968884 102.45001) (width 0.5) (layer B.Cu) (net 2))
 (segment (start 147.3 95.7) (end 147.3 94.65) (width 0.5) (layer B.Cu) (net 2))
 (segment (start 139.8875 98.647502) (end 139.819999 98.580001) (width 0.5) (layer B.Cu) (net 2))
 (segment (start 139.8875 99.7) (end 139.8875 98.647502) (width 0.5) (layer B.Cu) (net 2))
 (segment (start 138.814999 98.580001) (end 139.819999 98.580001) (width 0.5) (layer B.Cu) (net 2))
 (segment (start 139.819999 98.580001) (end 140.319999 98.580001) (width 0.5) (layer B.Cu) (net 2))
 (segment (start 149 92.95) (end 147.3 94.65) (width 0.5) (layer B.Cu) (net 2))
 (segment (start 149 92.5) (end 149 92.95) (width 0.5) (layer B.Cu) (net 2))
 (segment (start 148.6 96) (end 149 96) (width 0.25) (layer F.Cu) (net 12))
 (segment (start 144.8 92.2) (end 148.6 96) (width 0.25) (layer F.Cu) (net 12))
 (segment (start 143.75 92.2) (end 144.8 92.2) (width 0.25) (layer F.Cu) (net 12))
 (segment (start 132.8375 97.3375) (end 132.5 97) (width 0.2) (layer B.Cu) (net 11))
 (segment (start 135.1 97.3375) (end 132.8375 97.3375) (width 0.2) (layer B.Cu) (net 11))
 (via (at 133.9 90.7) (size 0.51) (drill 0.3) (layers F.Cu B.Cu) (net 11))
 (segment (start 132.5 97) (end 133.10104 97) (width 0.2) (layer F.Cu) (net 11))
 (segment (start 133.9 96.20104) (end 133.9 90.7) (width 0.2) (layer F.Cu) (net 11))
 (segment (start 133.10104 97) (end 133.9 96.20104) (width 0.2) (layer F.Cu) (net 11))
 (segment (start 140.044999 90.144999) (end 142.3 92.4) (width 0.2) (layer B.Cu) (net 11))
 (segment (start 133.9 90.7) (end 134.455001 90.144999) (width 0.2) (layer B.Cu) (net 11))
 (via (at 142.3 92.4) (size 0.51) (drill 0.3) (layers F.Cu B.Cu) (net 11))
 (segment (start 134.455001 90.144999) (end 140.044999 90.144999) (width 0.2) (layer B.Cu) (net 11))
 (segment (start 142.3 92.4) (end 142.3 90.75) (width 0.2) (layer F.Cu) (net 11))
 (segment (start 139 90.8) (end 139.1 90.7) (width 0.2) (layer B.Cu) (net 10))
 (segment (start 139 91.9625) (end 139 90.8) (width 0.2) (layer B.Cu) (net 10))
 (segment (start 134.35103 92.75001) (end 133.10104 94) (width 0.2) (layer B.Cu) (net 10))
 (segment (start 133.10104 94) (end 132.5 94) (width 0.2) (layer B.Cu) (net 10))
 (segment (start 138.21249 92.75001) (end 134.35103 92.75001) (width 0.2) (layer B.Cu) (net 10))
 (segment (start 139 91.9625) (end 138.21249 92.75001) (width 0.2) (layer B.Cu) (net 10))
 (segment (start 138.3 90.7625) (end 137.1 91.9625) (width 0.2) (layer B.Cu) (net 9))
 (segment (start 138.3 90.7) (end 138.3 90.7625) (width 0.2) (layer B.Cu) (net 9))
 (segment (start 133.5375 91.9625) (end 132.5 93) (width 0.2) (layer B.Cu) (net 9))
 (segment (start 137.1 91.9625) (end 133.5375 91.9625) (width 0.2) (layer B.Cu) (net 9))
 (segment (start 139.9 90.75) (end 140.7 90.75) (width 0.5) (layer F.Cu) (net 7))
 (segment (start 136.774999 97.900036) (end 137.375046 97.299989) (width 0.5) (layer F.Cu) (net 7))
 (segment (start 136.774999 99.225001) (end 136.774999 97.900036) (width 0.5) (layer F.Cu) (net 7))
 (segment (start 136.7 99.25) (end 136.75 99.25) (width 0.5) (layer F.Cu) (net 7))
 (segment (start 136.75 99.25) (end 136.774999 99.225001) (width 0.5) (layer F.Cu) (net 7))
 (segment (start 140.7 90.75) (end 140.649999 90.800001) (width 0.5) (layer F.Cu) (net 7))
 (segment (start 140.649999 96.350001) (end 139.700011 97.299989) (width 0.5) (layer F.Cu) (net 7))
 (segment (start 139.700011 97.299989) (end 137.375046 97.299989) (width 0.5) (layer F.Cu) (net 7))
 (via (at 140.649999 94.149999) (size 0.8) (drill 0.4) (layers F.Cu B.Cu) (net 7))
 (segment (start 140.45 94.349998) (end 140.649999 94.149999) (width 0.5) (layer B.Cu) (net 7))
 (segment (start 140.45 95.4) (end 140.45 94.349998) (width 0.5) (layer B.Cu) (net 7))
 (segment (start 140.649999 90.800001) (end 140.649999 94.149999) (width 0.5) (layer F.Cu) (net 7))
 (segment (start 140.649999 94.149999) (end 140.649999 96.350001) (width 0.5) (layer F.Cu) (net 7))
 (segment (start 137.1 93.8375) (end 139 93.8375) (width 0.5) (layer B.Cu) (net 7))
 (segment (start 140.3375 93.8375) (end 140.649999 94.149999) (width 0.5) (layer B.Cu) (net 7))
 (segment (start 139 93.8375) (end 140.3375 93.8375) (width 0.5) (layer B.Cu) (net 7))
 (segment (start 136.725 93.8375) (end 137.1 93.8375) (width 0.2) (layer B.Cu) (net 7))
 (segment (start 135.1 95.4625) (end 136.725 93.8375) (width 0.2) (layer B.Cu) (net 7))
 (segment (start 130.624999 93.579999) (end 131.204998 93) (width 0.5) (layer F.Cu) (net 7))
 (segment (start 130.624999 97.420001) (end 130.624999 93.579999) (width 0.5) (layer F.Cu) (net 7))
 (segment (start 131.204998 93) (end 131.5 93) (width 0.5) (layer F.Cu) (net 7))
 (segment (start 132.454998 99.25) (end 130.624999 97.420001) (width 0.5) (layer F.Cu) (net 7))
 (segment (start 136.7 99.25) (end 132.454998 99.25) (width 0.5) (layer F.Cu) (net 7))
 (segment (start 148 98.6) (end 148 102) (width 0.25) (layer F.Cu) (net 13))
 (segment (start 144.8 95.4) (end 148 98.6) (width 0.25) (layer F.Cu) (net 13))
 (segment (start 143.75 95.4) (end 144.8 95.4) (width 0.25) (layer F.Cu) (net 13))
 (segment (start 144.875001 96.275001) (end 144.875001 100.624999) (width 0.25) (layer F.Cu) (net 14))
 (segment (start 144.8 96.2) (end 144.875001 96.275001) (width 0.25) (layer F.Cu) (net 14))
 (segment (start 144.875001 100.624999) (end 143.5 102) (width 0.25) (layer F.Cu) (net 14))
 (segment (start 143.75 96.2) (end 144.8 96.2) (width 0.25) (layer F.Cu) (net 14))
 (segment (start 135.25 88.55) (end 135.1 88.4) (width 0.2) (layer F.Cu) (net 15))
 (segment (start 135.25 92.2) (end 135.25 88.55) (width 0.2) (layer F.Cu) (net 15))
 (segment (start 147.315002 93) (end 148 92.315002) (width 0.5) (layer B.Cu) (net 3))
 (segment (start 146.6 93) (end 147.315002 93) (width 0.5) (layer B.Cu) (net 3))
 (segment (start 148 90.0625) (end 146.5 88.5625) (width 0.5) (layer B.Cu) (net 3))
 (segment (start 148 92.315002) (end 148 90.0625) (width 0.5) (layer B.Cu) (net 3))
 (segment (start 146.5 88.5625) (end 146.5 88.5625) (width 0.5) (layer B.Cu) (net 3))
 (segment (start 149 88.5) (end 149 89.5) (width 0.5) (layer B.Cu) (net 3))
 (segment (start 148.4375 90.0625) (end 148 90.0625) (width 0.5) (layer B.Cu) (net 3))
 (segment (start 149 89.5) (end 148.4375 90.0625) (width 0.5) (layer B.Cu) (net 3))
 (segment (start 146.5 88.5625) (end 146.5 88.5625) (width 0.5) (layer B.Cu) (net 3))
 (via (at 146.5 88.5625) (size 0.8) (drill 0.4) (layers F.Cu B.Cu) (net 3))
 (segment (start 143.7 94.65) (end 144.4 93.95) (width 0.5) (layer B.Cu) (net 6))
 (segment (start 143.7 97.5) (end 143.7 94.65) (width 0.5) (layer B.Cu) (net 6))
 (segment (start 144.845002 92.05) (end 144.4 92.05) (width 0.2) (layer B.Cu) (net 1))
 (segment (start 145.5 92.704998) (end 144.845002 92.05) (width 0.2) (layer B.Cu) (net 1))
 (segment (start 145.5 101.3) (end 145.5 92.704998) (width 0.2) (layer B.Cu) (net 1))
 (segment (start 146.6 90.5375) (end 146.5 90.4375) (width 0.5) (layer B.Cu) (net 4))
 (segment (start 146.6 92.05) (end 146.6 90.5375) (width 0.5) (layer B.Cu) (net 4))
 (segment (start 146.5 90.4375) (end 144.5 90.4375) (width 0.5) (layer B.Cu) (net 4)))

